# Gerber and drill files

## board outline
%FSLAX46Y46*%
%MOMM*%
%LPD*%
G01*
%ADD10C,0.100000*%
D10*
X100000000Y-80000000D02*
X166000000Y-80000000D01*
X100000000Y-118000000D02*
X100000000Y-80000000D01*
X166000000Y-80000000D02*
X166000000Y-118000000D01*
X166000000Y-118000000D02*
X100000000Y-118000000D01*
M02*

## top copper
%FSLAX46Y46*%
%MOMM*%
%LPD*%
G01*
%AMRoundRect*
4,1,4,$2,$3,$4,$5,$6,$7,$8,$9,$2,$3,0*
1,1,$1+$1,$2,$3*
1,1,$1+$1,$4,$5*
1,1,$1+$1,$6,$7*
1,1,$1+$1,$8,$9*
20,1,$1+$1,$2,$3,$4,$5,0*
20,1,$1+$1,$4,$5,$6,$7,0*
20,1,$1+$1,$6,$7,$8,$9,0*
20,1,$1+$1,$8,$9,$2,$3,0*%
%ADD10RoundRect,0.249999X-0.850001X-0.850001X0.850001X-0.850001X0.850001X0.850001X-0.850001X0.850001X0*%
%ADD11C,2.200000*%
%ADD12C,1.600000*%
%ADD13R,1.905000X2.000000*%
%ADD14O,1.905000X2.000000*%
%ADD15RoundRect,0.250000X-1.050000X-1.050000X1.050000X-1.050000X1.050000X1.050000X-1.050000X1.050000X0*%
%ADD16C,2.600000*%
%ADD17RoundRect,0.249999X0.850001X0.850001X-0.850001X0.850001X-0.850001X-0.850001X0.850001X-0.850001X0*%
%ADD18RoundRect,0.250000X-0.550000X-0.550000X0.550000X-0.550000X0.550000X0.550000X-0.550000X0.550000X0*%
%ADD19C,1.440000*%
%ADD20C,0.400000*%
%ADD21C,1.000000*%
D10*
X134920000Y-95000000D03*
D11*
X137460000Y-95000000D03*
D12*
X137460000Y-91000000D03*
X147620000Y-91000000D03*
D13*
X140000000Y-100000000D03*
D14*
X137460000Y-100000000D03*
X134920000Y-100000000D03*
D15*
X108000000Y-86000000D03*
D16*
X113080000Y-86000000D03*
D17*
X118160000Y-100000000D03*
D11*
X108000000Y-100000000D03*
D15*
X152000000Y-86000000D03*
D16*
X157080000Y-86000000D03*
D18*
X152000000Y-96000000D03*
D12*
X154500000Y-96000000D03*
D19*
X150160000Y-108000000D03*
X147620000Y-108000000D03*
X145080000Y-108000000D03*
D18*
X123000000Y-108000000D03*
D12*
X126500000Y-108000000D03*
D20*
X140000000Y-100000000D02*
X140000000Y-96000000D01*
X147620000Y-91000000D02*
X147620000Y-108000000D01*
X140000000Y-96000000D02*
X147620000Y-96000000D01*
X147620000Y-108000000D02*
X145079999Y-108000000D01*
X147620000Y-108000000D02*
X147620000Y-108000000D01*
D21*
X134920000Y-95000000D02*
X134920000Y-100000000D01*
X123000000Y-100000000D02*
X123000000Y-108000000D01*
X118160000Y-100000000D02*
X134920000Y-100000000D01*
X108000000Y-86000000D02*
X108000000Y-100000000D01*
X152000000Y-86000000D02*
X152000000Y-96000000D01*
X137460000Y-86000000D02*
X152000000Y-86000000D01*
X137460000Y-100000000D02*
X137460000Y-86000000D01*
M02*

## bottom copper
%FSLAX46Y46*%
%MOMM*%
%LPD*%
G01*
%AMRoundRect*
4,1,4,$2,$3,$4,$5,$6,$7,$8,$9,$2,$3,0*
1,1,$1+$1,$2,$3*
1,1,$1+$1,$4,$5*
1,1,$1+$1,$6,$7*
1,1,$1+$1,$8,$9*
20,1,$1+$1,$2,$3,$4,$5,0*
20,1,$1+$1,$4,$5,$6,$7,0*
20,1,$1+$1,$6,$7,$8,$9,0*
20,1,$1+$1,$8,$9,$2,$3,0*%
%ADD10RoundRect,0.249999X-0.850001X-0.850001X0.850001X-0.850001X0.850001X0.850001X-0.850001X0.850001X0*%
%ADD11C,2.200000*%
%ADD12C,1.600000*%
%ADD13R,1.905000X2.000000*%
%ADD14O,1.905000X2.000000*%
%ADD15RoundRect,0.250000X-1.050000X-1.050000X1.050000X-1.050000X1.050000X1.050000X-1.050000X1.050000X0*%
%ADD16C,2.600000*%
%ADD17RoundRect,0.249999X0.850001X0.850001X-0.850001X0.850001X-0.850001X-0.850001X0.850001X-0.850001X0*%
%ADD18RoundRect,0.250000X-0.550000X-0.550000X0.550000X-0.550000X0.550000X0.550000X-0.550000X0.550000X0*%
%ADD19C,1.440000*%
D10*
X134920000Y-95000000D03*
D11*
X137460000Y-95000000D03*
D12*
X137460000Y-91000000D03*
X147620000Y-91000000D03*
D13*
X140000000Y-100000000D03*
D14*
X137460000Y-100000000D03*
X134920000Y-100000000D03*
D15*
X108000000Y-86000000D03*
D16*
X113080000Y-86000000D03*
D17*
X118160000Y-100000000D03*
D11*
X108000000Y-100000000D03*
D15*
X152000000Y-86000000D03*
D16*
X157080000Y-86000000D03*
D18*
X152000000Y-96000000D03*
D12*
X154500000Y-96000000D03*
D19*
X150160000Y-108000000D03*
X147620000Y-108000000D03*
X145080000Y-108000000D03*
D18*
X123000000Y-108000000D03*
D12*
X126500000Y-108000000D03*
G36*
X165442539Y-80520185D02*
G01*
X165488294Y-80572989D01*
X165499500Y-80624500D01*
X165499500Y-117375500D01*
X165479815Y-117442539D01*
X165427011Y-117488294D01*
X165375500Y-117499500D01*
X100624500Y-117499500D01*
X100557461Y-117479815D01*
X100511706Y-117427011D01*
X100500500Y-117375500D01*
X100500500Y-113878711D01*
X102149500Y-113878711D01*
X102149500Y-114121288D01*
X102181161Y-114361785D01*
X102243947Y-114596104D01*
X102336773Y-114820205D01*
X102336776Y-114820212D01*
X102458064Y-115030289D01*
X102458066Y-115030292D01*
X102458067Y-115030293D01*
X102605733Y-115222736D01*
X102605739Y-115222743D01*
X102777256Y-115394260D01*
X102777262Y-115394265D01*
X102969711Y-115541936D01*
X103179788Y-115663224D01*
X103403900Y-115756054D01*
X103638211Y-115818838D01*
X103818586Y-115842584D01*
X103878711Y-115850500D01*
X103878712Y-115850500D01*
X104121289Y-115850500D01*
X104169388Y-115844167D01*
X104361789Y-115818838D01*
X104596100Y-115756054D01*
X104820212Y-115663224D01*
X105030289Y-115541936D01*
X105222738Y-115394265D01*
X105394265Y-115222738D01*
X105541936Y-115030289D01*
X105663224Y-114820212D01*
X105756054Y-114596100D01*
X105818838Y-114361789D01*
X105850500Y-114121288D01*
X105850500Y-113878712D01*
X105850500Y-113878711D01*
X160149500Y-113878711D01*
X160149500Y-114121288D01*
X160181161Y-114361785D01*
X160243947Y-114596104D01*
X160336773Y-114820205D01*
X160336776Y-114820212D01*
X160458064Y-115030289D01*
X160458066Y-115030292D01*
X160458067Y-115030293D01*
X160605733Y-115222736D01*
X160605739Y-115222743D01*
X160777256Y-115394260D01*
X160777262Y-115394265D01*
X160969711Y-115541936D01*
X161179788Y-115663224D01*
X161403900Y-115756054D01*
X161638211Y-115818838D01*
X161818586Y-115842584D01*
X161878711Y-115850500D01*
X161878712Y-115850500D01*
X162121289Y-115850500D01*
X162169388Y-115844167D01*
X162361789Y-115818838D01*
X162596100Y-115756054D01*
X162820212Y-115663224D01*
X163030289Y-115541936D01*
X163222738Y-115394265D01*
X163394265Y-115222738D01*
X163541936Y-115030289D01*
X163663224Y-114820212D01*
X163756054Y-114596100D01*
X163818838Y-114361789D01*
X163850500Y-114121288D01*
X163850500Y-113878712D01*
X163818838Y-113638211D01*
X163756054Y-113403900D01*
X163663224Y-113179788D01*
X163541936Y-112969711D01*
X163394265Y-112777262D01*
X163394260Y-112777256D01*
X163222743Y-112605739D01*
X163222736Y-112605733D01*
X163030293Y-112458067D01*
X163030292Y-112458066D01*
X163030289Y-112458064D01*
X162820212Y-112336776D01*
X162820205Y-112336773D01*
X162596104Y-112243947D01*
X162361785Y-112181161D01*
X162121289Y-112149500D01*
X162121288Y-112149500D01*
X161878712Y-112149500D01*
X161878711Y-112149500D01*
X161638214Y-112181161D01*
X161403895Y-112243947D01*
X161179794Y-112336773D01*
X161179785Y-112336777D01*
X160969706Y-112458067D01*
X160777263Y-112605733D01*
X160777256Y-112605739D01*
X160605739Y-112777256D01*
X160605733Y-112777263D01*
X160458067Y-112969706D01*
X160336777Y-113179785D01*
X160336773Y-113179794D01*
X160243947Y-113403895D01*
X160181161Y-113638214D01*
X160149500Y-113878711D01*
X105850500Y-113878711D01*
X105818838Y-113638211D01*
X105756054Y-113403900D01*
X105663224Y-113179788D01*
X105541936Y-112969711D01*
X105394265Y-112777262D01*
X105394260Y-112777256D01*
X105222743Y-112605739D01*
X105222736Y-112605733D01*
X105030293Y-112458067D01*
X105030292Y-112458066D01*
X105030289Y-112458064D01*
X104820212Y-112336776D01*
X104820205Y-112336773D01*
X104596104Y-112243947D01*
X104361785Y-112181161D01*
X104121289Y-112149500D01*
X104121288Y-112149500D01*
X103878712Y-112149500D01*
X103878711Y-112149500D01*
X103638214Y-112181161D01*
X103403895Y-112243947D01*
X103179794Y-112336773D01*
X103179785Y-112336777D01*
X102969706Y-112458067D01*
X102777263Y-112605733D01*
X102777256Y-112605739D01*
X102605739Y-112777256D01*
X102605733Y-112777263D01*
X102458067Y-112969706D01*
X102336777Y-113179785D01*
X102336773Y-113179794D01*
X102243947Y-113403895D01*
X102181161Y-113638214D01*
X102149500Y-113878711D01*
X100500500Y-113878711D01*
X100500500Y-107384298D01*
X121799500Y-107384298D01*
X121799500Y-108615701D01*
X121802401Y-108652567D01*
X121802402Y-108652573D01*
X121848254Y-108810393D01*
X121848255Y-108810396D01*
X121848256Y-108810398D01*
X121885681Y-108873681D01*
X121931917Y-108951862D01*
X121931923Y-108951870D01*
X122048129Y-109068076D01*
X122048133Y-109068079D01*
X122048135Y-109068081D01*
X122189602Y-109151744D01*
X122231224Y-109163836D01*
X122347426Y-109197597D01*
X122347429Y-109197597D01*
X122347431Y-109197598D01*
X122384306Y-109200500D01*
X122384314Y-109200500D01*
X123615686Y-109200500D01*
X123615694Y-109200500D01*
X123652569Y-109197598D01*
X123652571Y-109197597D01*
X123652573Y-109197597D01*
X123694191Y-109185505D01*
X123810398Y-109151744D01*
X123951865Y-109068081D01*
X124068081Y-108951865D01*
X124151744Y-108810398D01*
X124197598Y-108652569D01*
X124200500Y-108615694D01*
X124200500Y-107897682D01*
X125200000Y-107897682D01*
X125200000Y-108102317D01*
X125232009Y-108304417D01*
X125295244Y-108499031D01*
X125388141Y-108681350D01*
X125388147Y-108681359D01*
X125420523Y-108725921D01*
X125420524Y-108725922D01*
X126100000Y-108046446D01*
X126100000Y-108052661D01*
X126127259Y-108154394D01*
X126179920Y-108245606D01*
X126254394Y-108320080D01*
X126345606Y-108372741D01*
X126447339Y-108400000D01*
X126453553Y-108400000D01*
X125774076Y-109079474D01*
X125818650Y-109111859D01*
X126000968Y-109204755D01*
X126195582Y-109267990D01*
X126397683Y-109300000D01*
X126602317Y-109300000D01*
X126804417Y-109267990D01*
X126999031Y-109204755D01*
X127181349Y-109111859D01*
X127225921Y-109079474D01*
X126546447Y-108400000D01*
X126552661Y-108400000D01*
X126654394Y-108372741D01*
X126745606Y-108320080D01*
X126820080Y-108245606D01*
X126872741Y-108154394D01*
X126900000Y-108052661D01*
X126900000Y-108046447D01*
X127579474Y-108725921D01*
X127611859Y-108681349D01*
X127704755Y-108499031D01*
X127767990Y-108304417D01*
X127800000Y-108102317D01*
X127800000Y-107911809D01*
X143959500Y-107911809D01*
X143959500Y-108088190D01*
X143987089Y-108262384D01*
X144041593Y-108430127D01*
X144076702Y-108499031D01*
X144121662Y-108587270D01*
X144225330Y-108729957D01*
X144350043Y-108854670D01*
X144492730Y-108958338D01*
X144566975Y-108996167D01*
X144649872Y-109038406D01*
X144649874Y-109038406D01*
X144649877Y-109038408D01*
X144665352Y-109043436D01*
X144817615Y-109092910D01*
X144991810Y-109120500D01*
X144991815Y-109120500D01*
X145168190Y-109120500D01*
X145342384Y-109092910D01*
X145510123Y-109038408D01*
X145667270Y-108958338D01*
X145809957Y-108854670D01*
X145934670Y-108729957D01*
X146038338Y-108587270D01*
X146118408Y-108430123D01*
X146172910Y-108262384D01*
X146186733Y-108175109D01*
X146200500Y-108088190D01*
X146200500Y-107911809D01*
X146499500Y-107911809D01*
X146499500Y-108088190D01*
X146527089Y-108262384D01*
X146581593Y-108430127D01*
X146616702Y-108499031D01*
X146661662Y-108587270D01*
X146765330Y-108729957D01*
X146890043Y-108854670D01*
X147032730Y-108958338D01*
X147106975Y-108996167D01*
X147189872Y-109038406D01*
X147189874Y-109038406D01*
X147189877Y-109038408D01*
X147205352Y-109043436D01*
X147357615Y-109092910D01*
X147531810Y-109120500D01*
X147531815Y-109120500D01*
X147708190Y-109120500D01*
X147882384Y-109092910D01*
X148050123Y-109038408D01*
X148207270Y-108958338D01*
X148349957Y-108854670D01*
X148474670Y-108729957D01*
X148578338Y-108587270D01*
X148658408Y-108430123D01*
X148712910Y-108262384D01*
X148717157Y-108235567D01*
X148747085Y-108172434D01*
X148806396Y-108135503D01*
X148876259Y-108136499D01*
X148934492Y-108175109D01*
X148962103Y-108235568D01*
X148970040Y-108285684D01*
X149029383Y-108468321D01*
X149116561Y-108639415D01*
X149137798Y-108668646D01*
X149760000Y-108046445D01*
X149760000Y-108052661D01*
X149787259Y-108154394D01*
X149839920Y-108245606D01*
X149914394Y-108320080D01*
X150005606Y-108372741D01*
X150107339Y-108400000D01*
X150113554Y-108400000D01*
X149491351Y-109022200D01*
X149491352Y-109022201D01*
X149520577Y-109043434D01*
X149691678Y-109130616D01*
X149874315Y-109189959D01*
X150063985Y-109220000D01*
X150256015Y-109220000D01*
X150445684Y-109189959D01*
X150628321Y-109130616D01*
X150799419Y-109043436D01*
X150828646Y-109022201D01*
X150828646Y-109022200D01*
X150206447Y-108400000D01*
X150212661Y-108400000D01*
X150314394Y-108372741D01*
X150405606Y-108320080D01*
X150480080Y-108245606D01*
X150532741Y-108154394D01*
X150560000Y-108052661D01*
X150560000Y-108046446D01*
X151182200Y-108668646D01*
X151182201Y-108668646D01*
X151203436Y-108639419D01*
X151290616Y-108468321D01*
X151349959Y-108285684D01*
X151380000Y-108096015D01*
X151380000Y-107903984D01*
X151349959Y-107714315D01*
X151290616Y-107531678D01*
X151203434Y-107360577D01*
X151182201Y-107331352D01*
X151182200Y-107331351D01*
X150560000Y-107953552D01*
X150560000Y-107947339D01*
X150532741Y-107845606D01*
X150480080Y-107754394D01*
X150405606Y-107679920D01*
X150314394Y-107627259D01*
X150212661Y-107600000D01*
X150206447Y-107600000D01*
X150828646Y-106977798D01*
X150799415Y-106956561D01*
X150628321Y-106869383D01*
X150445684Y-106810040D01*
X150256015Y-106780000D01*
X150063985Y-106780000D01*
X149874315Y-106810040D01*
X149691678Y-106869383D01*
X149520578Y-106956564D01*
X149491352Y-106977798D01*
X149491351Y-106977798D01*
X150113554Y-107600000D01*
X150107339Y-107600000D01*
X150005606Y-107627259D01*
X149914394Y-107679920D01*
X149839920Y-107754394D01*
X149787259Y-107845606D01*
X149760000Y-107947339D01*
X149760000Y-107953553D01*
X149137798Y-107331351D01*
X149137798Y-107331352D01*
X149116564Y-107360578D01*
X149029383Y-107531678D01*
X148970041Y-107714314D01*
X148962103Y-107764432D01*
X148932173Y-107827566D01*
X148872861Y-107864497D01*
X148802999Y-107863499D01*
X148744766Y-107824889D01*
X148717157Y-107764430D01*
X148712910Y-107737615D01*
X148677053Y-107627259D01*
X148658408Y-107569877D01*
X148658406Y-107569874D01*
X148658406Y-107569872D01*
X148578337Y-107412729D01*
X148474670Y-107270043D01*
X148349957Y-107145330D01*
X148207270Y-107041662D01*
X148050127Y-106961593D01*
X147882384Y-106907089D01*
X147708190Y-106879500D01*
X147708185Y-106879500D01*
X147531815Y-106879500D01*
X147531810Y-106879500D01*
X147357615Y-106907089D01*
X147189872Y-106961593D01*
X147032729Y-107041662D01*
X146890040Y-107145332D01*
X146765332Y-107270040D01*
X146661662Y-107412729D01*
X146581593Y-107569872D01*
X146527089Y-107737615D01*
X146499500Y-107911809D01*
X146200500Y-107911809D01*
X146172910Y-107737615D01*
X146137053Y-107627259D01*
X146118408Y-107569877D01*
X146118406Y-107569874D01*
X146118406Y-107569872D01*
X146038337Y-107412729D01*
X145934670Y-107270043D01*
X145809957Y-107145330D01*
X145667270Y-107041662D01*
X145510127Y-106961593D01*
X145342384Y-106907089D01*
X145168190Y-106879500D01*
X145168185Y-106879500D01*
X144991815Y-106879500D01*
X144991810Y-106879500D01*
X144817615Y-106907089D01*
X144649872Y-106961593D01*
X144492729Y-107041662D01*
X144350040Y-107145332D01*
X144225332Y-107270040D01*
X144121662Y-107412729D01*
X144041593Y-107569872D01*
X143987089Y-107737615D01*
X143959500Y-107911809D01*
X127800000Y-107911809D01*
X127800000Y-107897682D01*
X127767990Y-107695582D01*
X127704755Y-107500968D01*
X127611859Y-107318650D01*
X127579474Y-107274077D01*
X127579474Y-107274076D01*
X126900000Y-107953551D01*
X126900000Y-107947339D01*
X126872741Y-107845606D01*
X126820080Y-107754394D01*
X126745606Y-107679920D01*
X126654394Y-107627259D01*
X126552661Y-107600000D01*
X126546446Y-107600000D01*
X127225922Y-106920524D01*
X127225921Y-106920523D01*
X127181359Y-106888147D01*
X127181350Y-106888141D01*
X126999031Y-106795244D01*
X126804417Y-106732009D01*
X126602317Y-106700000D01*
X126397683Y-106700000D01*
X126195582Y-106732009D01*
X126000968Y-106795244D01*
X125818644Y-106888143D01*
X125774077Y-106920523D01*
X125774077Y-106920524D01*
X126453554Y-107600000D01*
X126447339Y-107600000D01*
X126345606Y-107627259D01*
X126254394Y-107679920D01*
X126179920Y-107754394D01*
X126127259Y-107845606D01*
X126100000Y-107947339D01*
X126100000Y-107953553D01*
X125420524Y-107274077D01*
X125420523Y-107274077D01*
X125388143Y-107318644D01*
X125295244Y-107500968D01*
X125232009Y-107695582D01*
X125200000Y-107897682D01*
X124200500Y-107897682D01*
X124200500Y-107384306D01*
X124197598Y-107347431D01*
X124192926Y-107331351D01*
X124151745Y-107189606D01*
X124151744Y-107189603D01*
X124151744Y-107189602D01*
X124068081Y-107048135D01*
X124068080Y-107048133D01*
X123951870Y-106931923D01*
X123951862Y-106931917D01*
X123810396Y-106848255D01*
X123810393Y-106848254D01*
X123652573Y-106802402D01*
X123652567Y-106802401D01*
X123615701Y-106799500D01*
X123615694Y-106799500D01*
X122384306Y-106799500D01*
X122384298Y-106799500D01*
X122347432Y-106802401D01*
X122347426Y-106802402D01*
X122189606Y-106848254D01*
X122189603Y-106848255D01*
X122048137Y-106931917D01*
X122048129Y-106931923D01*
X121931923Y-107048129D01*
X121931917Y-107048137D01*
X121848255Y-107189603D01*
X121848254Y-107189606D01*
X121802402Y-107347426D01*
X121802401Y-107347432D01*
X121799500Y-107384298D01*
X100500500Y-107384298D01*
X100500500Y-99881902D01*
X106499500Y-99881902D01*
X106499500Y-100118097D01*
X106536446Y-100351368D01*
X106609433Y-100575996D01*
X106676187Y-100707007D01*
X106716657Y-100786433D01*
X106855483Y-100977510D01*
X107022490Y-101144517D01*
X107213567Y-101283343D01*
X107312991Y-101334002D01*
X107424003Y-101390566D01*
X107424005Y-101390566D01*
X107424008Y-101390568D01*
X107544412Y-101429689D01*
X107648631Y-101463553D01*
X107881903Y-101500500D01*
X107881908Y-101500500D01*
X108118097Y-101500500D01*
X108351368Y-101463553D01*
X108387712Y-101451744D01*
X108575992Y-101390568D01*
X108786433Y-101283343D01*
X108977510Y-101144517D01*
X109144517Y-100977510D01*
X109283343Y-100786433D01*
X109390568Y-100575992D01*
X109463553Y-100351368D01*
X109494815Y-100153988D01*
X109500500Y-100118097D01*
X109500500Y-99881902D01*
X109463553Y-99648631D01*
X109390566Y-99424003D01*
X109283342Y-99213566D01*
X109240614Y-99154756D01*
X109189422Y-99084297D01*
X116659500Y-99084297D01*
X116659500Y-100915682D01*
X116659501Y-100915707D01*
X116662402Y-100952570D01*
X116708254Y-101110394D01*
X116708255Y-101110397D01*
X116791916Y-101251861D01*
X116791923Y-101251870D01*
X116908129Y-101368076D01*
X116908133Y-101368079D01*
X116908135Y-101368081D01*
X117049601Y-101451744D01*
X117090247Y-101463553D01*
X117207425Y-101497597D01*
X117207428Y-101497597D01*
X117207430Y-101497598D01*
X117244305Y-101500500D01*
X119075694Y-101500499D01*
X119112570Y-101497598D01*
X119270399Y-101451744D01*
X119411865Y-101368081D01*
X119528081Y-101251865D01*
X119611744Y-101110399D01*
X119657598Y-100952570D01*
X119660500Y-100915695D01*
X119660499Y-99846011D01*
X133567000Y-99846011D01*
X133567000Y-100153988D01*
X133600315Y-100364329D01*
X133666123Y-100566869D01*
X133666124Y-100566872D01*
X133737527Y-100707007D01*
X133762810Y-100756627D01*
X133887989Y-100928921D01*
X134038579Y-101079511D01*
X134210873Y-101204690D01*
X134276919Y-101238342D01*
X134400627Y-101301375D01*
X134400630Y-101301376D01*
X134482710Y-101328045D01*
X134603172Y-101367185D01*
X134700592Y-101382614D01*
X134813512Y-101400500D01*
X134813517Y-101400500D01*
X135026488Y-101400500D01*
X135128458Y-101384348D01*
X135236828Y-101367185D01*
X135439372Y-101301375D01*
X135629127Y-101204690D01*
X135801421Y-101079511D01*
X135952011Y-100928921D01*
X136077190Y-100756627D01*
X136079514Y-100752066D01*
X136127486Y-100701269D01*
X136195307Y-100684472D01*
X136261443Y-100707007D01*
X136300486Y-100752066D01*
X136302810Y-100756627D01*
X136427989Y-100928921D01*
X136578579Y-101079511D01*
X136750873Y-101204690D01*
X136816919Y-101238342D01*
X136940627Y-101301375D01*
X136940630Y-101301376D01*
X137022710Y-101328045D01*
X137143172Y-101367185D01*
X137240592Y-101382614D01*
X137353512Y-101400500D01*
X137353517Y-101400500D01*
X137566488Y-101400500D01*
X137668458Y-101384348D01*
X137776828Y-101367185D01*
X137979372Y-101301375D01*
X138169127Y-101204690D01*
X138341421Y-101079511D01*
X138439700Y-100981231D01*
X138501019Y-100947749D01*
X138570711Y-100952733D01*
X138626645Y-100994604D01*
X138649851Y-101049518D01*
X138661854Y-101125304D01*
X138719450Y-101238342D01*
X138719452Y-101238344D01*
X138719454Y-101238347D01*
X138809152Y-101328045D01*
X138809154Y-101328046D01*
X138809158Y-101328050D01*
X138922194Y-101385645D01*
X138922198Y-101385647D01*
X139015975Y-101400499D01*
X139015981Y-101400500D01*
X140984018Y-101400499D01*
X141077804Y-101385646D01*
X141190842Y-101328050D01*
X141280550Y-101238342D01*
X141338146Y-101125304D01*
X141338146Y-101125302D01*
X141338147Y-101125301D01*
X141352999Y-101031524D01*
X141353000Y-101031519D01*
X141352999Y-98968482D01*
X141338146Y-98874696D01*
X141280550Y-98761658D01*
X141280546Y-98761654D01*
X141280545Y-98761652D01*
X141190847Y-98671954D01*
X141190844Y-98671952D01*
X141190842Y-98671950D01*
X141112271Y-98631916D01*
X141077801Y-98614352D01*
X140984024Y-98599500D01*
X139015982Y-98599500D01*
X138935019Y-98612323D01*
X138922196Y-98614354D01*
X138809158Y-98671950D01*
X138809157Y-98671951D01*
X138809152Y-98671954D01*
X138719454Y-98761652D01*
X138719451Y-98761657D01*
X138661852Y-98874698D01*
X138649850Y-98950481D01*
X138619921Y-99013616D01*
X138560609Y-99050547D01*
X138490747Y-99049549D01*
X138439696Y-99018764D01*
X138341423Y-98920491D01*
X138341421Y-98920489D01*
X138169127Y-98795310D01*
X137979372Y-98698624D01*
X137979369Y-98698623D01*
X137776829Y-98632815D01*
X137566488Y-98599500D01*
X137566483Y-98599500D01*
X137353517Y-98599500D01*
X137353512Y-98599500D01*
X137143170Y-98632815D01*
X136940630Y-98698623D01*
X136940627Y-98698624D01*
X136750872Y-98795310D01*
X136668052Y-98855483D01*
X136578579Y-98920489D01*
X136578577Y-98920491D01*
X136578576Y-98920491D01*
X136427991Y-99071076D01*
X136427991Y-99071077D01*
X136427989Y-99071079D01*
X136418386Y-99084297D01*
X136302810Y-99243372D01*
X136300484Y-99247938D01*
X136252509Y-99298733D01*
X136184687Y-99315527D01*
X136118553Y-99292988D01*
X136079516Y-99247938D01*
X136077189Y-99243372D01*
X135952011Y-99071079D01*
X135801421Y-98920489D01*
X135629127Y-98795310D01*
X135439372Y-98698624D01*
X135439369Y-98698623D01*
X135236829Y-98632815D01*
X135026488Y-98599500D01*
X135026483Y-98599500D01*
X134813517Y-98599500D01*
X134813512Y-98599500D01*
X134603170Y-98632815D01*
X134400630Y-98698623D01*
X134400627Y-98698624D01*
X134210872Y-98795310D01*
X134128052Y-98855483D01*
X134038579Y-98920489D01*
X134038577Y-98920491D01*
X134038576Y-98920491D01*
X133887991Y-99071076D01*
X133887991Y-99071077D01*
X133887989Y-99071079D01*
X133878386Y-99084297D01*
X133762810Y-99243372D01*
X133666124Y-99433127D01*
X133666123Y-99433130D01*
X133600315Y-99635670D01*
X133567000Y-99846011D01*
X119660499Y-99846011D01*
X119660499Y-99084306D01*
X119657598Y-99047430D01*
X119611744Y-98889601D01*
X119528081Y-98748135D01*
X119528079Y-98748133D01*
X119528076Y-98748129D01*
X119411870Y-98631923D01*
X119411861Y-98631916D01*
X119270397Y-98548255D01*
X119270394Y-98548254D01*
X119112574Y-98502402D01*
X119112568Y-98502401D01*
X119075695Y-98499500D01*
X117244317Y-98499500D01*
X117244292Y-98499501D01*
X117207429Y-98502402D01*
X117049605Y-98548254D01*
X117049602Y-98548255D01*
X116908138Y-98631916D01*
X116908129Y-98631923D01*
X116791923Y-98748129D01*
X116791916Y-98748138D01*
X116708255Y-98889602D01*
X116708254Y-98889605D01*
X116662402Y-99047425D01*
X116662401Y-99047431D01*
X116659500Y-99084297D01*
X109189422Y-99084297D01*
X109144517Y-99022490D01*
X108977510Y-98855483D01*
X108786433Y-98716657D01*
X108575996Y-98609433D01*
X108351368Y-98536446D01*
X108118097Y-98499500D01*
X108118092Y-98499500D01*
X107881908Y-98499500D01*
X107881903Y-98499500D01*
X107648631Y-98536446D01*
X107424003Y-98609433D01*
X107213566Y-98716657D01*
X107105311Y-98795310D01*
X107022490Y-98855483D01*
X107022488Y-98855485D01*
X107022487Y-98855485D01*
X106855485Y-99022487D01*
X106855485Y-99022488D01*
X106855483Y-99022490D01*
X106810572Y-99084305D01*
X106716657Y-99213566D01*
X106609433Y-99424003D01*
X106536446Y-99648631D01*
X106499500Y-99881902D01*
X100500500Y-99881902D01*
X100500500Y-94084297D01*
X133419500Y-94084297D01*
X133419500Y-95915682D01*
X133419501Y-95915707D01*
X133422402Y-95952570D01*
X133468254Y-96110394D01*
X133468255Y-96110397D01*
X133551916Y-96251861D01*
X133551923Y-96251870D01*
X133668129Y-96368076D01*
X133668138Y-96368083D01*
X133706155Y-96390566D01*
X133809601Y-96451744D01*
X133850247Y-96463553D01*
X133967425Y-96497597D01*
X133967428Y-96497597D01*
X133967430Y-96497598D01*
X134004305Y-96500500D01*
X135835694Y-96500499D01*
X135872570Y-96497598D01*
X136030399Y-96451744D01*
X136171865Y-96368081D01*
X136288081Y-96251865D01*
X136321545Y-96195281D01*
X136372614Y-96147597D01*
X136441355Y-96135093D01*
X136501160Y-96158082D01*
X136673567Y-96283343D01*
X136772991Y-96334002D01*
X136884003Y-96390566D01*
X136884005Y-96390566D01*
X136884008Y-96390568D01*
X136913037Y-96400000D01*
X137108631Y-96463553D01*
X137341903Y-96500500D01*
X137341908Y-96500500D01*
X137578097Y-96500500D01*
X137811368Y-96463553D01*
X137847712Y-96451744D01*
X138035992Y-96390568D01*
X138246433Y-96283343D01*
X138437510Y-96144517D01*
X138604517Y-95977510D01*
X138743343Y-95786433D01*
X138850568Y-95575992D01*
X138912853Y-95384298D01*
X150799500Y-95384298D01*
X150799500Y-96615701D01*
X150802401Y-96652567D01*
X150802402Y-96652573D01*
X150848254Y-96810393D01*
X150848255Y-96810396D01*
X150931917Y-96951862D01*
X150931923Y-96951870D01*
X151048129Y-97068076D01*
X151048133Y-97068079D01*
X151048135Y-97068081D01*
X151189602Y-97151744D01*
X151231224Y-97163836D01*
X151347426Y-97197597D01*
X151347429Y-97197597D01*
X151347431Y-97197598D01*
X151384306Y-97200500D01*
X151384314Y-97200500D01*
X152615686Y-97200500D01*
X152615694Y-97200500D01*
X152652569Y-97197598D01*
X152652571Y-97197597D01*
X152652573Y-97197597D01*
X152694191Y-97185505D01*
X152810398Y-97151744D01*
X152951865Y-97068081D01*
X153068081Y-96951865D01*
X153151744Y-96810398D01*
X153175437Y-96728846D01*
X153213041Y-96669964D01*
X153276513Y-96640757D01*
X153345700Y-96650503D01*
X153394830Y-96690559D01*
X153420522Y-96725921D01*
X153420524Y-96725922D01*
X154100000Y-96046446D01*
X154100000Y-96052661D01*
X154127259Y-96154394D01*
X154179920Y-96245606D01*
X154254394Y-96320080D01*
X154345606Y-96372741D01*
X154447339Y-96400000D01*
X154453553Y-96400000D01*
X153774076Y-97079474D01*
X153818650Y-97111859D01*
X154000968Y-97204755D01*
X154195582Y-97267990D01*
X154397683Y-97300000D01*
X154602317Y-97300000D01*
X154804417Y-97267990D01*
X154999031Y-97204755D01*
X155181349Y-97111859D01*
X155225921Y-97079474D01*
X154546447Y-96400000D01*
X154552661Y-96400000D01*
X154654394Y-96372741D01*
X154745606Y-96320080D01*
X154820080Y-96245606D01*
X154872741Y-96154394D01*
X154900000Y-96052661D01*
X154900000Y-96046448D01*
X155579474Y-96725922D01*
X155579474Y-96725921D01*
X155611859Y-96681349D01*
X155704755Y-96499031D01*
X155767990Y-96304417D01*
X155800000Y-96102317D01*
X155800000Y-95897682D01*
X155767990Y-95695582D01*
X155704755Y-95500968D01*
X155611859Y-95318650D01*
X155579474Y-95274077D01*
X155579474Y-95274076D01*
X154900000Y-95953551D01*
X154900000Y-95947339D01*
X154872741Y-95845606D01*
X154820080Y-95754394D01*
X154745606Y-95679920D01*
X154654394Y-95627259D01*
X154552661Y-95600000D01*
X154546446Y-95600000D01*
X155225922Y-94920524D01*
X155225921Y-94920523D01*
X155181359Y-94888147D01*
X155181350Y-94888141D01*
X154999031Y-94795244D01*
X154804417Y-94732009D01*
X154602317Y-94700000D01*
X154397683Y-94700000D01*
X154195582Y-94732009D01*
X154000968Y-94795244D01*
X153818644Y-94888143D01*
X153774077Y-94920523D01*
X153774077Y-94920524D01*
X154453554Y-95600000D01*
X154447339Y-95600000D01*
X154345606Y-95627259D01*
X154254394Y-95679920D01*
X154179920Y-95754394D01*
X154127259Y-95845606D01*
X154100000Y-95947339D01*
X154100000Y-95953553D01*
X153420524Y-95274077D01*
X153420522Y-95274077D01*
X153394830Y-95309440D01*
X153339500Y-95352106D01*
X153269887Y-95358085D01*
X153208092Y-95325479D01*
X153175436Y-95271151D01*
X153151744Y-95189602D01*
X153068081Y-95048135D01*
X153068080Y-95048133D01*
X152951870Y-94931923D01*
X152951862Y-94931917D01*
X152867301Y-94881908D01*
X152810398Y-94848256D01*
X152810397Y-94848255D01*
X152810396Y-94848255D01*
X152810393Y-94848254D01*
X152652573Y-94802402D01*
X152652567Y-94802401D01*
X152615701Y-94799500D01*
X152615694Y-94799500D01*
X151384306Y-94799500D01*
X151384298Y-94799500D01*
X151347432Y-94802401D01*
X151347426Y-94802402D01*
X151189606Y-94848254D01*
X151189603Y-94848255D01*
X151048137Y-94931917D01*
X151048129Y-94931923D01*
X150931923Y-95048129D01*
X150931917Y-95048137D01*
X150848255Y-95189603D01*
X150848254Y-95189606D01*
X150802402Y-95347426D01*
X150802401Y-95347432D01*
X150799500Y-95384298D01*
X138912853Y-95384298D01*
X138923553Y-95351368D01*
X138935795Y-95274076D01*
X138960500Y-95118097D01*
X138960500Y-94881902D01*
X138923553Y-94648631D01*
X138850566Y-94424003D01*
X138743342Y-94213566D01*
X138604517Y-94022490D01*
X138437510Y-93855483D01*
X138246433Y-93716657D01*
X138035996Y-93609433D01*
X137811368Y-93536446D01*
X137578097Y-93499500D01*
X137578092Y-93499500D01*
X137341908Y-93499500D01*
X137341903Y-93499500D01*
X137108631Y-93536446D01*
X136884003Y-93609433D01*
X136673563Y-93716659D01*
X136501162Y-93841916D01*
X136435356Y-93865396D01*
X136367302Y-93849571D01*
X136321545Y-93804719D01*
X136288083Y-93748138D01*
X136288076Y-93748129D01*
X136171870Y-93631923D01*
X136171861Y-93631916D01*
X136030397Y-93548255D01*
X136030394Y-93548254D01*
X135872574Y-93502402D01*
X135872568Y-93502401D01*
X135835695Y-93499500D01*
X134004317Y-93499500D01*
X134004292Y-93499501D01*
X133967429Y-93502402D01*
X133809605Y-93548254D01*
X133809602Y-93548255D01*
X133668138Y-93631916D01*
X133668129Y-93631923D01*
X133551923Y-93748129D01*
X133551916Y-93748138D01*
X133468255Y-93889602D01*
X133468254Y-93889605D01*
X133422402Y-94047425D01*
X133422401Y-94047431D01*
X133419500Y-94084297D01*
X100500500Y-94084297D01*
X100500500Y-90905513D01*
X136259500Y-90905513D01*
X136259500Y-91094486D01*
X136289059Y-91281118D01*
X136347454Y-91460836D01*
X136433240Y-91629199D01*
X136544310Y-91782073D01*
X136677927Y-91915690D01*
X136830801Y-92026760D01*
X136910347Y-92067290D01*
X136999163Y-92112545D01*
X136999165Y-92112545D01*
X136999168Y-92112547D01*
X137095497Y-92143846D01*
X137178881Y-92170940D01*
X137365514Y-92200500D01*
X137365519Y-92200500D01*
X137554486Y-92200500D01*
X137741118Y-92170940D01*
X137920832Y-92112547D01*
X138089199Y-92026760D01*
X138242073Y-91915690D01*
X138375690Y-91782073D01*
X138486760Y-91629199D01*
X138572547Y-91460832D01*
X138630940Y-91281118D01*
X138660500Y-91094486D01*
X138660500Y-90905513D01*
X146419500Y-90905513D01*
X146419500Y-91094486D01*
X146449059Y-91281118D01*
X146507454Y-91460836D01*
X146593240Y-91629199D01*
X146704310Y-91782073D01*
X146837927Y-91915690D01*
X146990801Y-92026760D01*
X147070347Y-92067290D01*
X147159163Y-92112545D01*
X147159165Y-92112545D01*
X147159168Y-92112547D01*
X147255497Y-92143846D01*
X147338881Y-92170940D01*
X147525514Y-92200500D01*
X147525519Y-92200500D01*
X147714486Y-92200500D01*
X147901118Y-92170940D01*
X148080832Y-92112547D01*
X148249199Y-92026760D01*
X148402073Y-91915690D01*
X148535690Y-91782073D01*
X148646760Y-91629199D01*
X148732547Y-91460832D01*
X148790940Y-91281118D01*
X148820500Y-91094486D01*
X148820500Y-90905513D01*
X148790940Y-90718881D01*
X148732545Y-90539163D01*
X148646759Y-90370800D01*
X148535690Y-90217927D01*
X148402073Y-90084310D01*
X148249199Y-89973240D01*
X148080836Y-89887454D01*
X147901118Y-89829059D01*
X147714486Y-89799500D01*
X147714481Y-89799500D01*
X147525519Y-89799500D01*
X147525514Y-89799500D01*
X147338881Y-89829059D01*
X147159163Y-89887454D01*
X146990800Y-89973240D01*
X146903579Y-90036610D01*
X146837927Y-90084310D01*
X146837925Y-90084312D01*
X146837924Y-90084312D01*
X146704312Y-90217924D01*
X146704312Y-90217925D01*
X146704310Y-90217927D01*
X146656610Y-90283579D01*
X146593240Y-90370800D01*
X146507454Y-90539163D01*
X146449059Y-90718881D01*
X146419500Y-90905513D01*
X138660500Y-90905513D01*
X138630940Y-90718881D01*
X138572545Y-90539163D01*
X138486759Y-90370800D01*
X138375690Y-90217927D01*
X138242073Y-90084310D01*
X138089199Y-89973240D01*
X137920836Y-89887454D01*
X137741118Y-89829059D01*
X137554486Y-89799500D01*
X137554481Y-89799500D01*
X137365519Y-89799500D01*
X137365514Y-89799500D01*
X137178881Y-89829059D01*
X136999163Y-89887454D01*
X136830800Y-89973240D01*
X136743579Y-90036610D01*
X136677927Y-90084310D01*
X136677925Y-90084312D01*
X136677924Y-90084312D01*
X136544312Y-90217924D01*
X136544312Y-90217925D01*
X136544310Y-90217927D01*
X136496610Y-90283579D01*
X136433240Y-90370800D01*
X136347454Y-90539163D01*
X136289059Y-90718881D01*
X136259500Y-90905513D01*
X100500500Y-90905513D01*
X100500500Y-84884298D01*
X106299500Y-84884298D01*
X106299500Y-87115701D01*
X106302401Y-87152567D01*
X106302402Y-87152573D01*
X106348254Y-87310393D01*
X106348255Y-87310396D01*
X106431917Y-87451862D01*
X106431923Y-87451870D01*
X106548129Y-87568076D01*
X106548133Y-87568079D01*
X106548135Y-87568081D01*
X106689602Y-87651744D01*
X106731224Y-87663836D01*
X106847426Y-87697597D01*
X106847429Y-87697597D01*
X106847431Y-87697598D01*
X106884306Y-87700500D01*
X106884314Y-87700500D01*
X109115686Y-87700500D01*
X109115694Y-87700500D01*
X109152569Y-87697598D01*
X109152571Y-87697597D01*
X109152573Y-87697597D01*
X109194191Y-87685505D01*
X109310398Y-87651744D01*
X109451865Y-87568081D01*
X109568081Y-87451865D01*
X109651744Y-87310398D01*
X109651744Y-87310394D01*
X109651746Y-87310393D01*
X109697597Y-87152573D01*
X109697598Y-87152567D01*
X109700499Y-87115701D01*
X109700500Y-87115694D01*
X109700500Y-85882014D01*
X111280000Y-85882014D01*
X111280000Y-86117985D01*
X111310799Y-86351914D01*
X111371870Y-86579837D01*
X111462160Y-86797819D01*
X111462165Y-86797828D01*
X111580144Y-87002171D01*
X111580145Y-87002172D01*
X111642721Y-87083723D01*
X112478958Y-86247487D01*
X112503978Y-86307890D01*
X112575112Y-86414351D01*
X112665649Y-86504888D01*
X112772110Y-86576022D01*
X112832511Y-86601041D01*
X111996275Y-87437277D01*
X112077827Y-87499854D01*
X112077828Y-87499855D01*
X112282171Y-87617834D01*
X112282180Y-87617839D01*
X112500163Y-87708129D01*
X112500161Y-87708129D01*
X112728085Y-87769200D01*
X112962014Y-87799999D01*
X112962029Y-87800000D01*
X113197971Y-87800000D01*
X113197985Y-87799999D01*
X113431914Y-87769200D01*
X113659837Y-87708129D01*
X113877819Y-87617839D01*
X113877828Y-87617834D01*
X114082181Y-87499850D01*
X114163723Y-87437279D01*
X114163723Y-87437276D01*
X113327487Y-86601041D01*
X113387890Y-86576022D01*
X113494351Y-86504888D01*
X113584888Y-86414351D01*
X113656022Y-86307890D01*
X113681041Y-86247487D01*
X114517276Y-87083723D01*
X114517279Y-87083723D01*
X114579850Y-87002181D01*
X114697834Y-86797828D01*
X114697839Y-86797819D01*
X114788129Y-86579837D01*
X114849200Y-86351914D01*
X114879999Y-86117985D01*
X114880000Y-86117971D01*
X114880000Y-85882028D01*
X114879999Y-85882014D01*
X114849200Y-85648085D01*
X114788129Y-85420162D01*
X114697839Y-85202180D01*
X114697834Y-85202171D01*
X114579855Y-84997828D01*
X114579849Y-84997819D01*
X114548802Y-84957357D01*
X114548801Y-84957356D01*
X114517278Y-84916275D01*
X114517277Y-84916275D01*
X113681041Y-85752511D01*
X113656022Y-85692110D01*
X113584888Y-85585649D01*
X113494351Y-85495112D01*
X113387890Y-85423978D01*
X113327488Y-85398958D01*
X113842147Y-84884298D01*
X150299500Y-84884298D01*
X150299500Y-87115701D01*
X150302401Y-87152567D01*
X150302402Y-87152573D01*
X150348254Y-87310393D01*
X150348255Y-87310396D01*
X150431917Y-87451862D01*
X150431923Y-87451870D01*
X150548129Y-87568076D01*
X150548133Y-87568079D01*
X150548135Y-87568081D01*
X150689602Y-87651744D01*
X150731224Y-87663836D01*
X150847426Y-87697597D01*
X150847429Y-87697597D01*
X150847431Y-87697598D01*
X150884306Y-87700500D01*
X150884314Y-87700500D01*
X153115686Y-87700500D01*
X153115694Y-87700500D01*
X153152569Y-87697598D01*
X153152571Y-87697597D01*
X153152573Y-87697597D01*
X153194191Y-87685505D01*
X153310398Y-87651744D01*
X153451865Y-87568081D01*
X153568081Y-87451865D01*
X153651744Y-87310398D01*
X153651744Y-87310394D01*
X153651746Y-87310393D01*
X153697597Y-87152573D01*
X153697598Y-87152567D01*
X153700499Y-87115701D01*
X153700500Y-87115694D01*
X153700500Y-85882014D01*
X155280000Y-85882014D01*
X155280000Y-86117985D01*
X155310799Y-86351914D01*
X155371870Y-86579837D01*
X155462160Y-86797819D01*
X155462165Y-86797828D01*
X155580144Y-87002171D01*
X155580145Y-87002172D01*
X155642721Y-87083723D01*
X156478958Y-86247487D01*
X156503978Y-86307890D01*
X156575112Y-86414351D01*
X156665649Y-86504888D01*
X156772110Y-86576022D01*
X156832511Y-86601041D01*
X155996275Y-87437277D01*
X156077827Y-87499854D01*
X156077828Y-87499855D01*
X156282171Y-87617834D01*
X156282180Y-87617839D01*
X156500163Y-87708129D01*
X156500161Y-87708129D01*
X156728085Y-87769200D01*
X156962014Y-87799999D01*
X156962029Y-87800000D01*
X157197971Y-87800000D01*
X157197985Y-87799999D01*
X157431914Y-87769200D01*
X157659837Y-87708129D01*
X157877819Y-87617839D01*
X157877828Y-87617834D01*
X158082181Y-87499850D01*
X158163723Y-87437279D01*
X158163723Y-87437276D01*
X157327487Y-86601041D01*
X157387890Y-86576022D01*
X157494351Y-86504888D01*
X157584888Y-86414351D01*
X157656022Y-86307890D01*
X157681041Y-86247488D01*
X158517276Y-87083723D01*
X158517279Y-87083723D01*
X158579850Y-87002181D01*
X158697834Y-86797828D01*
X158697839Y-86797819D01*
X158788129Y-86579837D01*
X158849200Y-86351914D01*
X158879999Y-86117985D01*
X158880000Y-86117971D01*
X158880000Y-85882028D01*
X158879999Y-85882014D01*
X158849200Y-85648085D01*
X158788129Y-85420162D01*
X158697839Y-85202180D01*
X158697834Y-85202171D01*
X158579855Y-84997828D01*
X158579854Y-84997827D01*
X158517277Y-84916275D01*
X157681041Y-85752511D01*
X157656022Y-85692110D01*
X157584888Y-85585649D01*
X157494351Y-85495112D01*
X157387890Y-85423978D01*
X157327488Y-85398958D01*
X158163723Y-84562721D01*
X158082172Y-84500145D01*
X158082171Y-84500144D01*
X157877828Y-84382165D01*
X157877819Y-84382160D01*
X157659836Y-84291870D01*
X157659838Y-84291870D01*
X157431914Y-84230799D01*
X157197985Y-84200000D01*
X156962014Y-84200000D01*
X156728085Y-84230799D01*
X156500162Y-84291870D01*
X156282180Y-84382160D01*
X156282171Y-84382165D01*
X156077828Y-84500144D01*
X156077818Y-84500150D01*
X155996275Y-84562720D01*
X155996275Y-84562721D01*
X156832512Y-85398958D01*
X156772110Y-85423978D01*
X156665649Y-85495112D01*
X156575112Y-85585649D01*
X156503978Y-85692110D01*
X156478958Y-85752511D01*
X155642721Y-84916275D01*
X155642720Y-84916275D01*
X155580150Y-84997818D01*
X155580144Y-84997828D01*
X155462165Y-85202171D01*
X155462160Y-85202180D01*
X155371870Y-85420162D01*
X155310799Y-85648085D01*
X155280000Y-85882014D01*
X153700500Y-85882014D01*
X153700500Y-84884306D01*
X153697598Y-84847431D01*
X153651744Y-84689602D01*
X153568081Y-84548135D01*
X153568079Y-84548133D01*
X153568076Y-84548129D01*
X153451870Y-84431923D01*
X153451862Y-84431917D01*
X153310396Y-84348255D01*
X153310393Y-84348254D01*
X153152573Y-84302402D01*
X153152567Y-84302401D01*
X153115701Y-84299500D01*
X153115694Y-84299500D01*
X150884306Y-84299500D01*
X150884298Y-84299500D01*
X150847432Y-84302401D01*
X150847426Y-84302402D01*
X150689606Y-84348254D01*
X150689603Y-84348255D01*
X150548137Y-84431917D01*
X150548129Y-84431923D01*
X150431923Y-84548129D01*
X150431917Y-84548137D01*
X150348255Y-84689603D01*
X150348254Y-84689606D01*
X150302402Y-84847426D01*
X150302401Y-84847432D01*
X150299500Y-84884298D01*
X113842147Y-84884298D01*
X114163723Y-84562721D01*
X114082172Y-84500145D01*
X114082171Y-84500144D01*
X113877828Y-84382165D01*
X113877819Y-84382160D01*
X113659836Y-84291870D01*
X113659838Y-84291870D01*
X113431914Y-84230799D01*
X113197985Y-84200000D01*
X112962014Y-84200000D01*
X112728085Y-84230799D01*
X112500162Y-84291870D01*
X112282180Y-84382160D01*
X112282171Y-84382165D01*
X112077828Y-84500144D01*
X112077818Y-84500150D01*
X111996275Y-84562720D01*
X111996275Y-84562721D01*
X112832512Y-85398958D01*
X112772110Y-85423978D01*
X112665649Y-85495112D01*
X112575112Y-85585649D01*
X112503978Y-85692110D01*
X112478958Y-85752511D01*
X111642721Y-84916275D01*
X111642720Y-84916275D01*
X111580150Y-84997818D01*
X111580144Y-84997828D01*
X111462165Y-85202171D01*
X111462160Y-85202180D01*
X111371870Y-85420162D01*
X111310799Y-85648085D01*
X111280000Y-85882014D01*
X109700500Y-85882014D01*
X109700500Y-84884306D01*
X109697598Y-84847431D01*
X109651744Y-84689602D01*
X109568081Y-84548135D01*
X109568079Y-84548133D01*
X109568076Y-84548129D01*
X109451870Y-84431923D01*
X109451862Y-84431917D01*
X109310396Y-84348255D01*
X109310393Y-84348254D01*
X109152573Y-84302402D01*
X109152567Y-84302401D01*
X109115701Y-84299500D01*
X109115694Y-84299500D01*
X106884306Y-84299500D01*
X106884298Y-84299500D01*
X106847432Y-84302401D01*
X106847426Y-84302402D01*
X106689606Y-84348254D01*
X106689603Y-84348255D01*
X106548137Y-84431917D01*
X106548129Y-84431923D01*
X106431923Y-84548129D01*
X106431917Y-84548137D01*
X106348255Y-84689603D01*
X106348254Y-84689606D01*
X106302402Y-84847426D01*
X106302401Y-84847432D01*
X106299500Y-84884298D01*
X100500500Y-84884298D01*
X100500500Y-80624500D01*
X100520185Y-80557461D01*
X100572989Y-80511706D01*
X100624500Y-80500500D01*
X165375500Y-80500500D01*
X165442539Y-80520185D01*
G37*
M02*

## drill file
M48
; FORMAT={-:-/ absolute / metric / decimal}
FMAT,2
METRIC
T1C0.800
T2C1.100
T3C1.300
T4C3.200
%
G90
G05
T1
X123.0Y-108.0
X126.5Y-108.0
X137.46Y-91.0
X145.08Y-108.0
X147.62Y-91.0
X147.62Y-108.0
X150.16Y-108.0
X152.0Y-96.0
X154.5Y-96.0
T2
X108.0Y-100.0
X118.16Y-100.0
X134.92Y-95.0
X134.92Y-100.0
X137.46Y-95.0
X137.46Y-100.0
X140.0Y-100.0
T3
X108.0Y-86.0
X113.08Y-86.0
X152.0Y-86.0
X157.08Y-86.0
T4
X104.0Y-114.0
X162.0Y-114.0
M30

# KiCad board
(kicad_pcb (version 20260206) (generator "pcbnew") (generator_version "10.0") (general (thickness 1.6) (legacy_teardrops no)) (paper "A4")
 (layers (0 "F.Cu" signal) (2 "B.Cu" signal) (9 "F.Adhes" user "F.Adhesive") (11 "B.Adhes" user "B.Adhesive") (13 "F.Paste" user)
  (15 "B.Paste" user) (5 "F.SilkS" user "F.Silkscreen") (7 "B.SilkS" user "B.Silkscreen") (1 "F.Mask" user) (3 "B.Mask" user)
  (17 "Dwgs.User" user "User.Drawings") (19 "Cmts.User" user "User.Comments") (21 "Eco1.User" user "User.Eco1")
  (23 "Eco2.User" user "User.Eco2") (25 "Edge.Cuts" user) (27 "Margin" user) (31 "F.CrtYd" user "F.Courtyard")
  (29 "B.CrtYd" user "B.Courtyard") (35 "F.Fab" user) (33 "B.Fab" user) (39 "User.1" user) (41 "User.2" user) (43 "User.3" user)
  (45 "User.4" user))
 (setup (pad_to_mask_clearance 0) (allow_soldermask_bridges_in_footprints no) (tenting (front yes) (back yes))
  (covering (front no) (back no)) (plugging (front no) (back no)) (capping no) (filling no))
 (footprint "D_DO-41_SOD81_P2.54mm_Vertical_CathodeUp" (layer "F.Cu") (at 134.92 95)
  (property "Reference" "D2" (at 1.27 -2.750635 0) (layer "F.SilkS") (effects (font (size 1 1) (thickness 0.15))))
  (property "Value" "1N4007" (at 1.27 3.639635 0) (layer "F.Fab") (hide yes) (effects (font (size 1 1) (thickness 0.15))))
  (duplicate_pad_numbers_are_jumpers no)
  (pad "1" thru_hole roundrect (at 0 0) (size 2.2 2.2) (drill 1.1) (layers "*.Cu" "*.Mask") (remove_unused_layers no)
   (roundrect_rratio 0.113636) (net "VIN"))
  (pad "2" thru_hole circle (at 2.54 0) (size 2.2 2.2) (drill 1.1) (layers "*.Cu" "*.Mask") (remove_unused_layers no) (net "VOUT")))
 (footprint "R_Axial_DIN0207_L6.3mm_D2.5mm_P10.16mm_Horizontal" (layer "F.Cu") (at 137.46 91)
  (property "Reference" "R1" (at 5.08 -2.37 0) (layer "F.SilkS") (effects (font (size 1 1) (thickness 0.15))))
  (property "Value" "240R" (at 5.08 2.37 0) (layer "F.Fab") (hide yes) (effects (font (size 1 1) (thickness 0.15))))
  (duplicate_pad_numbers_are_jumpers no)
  (pad "1" thru_hole circle (at 0 0) (size 1.6 1.6) (drill 0.8) (layers "*.Cu" "*.Mask") (remove_unused_layers no) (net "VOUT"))
  (pad "2" thru_hole circle (at 10.16 0) (size 1.6 1.6) (drill 0.8) (layers "*.Cu" "*.Mask") (remove_unused_layers no) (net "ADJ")))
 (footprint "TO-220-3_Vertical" (layer "F.Cu") (at 140 100 180)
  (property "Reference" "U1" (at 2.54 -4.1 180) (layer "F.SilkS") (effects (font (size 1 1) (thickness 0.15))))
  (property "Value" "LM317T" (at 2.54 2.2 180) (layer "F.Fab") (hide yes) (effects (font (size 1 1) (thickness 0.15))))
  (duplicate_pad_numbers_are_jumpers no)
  (pad "1" thru_hole rect (at 0 0 180) (size 1.905 2) (drill 1.1) (layers "*.Cu" "*.Mask") (remove_unused_layers no) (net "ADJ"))
  (pad "2" thru_hole oval (at 2.54 0 180) (size 1.905 2) (drill 1.1) (layers "*.Cu" "*.Mask") (remove_unused_layers no) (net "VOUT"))
  (pad "3" thru_hole oval (at 5.08 0 180) (size 1.905 2) (drill 1.1) (layers "*.Cu" "*.Mask") (remove_unused_layers no) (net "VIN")))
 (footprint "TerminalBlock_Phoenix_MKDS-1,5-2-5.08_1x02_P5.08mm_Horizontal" (layer "F.Cu") (at 108 86)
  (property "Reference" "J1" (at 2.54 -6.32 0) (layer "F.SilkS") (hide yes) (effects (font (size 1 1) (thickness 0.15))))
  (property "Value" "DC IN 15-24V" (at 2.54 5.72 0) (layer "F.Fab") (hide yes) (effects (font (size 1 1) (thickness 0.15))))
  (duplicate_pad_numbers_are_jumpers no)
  (pad "1" thru_hole roundrect (at 0 0) (size 2.6 2.6) (drill 1.3) (layers "*.Cu" "*.Mask") (remove_unused_layers no)
   (roundrect_rratio 0.096154) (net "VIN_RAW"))
  (pad "2" thru_hole circle (at 5.08 0) (size 2.6 2.6) (drill 1.3) (layers "*.Cu" "*.Mask") (remove_unused_layers no) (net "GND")))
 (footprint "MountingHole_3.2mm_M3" (layer "F.Cu") (at 162 114)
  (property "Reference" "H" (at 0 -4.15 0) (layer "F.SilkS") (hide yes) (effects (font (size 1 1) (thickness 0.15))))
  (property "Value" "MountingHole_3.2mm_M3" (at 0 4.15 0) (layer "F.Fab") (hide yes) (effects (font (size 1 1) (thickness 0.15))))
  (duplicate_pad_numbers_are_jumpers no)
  (pad "" np_thru_hole circle (at 0 0) (size 3.2 3.2) (drill 3.2) (layers "*.Cu" "*.Mask")))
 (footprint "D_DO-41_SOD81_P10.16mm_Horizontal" (layer "F.Cu") (at 118.16 100 180)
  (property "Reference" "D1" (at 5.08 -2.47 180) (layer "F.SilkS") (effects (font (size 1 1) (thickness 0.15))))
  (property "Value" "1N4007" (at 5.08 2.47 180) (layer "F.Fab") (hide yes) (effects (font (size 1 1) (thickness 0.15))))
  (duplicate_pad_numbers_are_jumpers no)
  (pad "1" thru_hole roundrect (at 0 0 180) (size 2.2 2.2) (drill 1.1) (layers "*.Cu" "*.Mask") (remove_unused_layers no)
   (roundrect_rratio 0.113636) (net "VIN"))
  (pad "2" thru_hole circle (at 10.16 0 180) (size 2.2 2.2) (drill 1.1) (layers "*.Cu" "*.Mask") (remove_unused_layers no) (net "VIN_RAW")))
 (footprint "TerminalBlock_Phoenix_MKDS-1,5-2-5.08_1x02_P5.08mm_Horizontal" (layer "F.Cu") (at 152 86)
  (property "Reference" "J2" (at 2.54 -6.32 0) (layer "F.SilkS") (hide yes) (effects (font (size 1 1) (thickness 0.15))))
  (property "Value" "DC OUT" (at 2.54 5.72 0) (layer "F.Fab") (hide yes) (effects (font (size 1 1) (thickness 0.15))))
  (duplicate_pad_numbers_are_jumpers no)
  (pad "1" thru_hole roundrect (at 0 0) (size 2.6 2.6) (drill 1.3) (layers "*.Cu" "*.Mask") (remove_unused_layers no)
   (roundrect_rratio 0.096154) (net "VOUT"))
  (pad "2" thru_hole circle (at 5.08 0) (size 2.6 2.6) (drill 1.3) (layers "*.Cu" "*.Mask") (remove_unused_layers no) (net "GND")))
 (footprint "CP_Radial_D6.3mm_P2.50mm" (layer "F.Cu") (at 152 96)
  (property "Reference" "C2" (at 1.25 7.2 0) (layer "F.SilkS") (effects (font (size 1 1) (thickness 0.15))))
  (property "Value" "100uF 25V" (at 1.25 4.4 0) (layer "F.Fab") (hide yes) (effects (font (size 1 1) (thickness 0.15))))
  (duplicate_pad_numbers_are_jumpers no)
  (pad "1" thru_hole roundrect (at 0 0) (size 1.6 1.6) (drill 0.8) (layers "*.Cu" "*.Mask") (remove_unused_layers no)
   (roundrect_rratio 0.15625) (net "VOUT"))
  (pad "2" thru_hole circle (at 2.5 0) (size 1.6 1.6) (drill 0.8) (layers "*.Cu" "*.Mask") (remove_unused_layers no) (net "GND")))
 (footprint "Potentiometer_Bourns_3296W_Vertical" (layer "F.Cu") (at 150.16 108)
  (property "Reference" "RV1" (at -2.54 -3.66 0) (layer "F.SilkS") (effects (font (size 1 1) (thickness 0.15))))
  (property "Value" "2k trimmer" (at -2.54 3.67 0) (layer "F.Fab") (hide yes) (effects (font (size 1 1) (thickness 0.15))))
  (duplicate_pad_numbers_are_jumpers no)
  (pad "1" thru_hole circle (at 0 0) (size 1.44 1.44) (drill 0.8) (layers "*.Cu" "*.Mask") (remove_unused_layers no) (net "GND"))
  (pad "2" thru_hole circle (at -2.54 0) (size 1.44 1.44) (drill 0.8) (layers "*.Cu" "*.Mask") (remove_unused_layers no) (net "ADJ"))
  (pad "3" thru_hole circle (at -5.08 0) (size 1.44 1.44) (drill 0.8) (layers "*.Cu" "*.Mask") (remove_unused_layers no) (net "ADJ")))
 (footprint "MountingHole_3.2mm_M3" (layer "F.Cu") (at 104 114)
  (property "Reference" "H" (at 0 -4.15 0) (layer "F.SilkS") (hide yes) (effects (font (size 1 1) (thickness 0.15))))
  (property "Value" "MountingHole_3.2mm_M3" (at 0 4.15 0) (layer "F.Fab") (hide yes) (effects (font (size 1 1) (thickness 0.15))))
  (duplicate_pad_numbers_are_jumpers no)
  (pad "" np_thru_hole circle (at 0 0) (size 3.2 3.2) (drill 3.2) (layers "*.Cu" "*.Mask")))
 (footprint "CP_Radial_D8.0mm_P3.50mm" (layer "F.Cu") (at 123 108)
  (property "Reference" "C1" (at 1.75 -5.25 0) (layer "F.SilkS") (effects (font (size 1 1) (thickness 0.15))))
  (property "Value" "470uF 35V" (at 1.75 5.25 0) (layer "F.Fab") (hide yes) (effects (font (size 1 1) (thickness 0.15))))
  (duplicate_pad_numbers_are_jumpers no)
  (pad "1" thru_hole roundrect (at 0 0) (size 1.6 1.6) (drill 0.8) (layers "*.Cu" "*.Mask") (remove_unused_layers no)
   (roundrect_rratio 0.15625) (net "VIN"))
  (pad "2" thru_hole circle (at 3.5 0) (size 1.6 1.6) (drill 0.8) (layers "*.Cu" "*.Mask") (remove_unused_layers no) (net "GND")))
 (gr_line (start 100 80) (end 166 80) (stroke (width 0.1) (type default)) (layer "Edge.Cuts"))
 (gr_line (start 100 118) (end 100 80) (stroke (width 0.1) (type default)) (layer "Edge.Cuts"))
 (gr_line (start 166 80) (end 166 118) (stroke (width 0.1) (type default)) (layer "Edge.Cuts"))
 (gr_line (start 166 118) (end 100 118) (stroke (width 0.1) (type default)) (layer "Edge.Cuts"))
 (segment (start 140 100) (end 140 96) (width 0.4) (layer "F.Cu") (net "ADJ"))
 (segment (start 147.62 91) (end 147.62 108) (width 0.4) (layer "F.Cu") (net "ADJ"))
 (segment (start 140 96) (end 147.62 96) (width 0.4) (layer "F.Cu") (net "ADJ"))
 (segment (start 147.62 108) (end 145.079999 108) (width 0.4) (layer "F.Cu") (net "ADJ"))
 (segment (start 147.62 108) (end 147.62 108) (width 0.4) (layer "F.Cu") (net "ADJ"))
 (segment (start 134.92 95) (end 134.92 100) (width 1) (layer "F.Cu") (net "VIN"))
 (segment (start 123 100) (end 123 108) (width 1) (layer "F.Cu") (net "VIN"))
 (segment (start 118.16 100) (end 134.92 100) (width 1) (layer "F.Cu") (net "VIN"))
 (segment (start 108 86) (end 108 100) (width 1) (layer "F.Cu") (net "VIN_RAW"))
 (segment (start 152 86) (end 152 96) (width 1) (layer "F.Cu") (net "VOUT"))
 (segment (start 137.46 86) (end 152 86) (width 1) (layer "F.Cu") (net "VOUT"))
 (segment (start 137.46 100) (end 137.46 86) (width 1) (layer "F.Cu") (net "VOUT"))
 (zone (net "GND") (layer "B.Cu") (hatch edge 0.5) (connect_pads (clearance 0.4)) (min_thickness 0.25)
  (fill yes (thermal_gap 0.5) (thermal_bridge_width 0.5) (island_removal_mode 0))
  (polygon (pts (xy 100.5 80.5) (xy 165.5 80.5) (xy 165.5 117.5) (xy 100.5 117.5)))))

